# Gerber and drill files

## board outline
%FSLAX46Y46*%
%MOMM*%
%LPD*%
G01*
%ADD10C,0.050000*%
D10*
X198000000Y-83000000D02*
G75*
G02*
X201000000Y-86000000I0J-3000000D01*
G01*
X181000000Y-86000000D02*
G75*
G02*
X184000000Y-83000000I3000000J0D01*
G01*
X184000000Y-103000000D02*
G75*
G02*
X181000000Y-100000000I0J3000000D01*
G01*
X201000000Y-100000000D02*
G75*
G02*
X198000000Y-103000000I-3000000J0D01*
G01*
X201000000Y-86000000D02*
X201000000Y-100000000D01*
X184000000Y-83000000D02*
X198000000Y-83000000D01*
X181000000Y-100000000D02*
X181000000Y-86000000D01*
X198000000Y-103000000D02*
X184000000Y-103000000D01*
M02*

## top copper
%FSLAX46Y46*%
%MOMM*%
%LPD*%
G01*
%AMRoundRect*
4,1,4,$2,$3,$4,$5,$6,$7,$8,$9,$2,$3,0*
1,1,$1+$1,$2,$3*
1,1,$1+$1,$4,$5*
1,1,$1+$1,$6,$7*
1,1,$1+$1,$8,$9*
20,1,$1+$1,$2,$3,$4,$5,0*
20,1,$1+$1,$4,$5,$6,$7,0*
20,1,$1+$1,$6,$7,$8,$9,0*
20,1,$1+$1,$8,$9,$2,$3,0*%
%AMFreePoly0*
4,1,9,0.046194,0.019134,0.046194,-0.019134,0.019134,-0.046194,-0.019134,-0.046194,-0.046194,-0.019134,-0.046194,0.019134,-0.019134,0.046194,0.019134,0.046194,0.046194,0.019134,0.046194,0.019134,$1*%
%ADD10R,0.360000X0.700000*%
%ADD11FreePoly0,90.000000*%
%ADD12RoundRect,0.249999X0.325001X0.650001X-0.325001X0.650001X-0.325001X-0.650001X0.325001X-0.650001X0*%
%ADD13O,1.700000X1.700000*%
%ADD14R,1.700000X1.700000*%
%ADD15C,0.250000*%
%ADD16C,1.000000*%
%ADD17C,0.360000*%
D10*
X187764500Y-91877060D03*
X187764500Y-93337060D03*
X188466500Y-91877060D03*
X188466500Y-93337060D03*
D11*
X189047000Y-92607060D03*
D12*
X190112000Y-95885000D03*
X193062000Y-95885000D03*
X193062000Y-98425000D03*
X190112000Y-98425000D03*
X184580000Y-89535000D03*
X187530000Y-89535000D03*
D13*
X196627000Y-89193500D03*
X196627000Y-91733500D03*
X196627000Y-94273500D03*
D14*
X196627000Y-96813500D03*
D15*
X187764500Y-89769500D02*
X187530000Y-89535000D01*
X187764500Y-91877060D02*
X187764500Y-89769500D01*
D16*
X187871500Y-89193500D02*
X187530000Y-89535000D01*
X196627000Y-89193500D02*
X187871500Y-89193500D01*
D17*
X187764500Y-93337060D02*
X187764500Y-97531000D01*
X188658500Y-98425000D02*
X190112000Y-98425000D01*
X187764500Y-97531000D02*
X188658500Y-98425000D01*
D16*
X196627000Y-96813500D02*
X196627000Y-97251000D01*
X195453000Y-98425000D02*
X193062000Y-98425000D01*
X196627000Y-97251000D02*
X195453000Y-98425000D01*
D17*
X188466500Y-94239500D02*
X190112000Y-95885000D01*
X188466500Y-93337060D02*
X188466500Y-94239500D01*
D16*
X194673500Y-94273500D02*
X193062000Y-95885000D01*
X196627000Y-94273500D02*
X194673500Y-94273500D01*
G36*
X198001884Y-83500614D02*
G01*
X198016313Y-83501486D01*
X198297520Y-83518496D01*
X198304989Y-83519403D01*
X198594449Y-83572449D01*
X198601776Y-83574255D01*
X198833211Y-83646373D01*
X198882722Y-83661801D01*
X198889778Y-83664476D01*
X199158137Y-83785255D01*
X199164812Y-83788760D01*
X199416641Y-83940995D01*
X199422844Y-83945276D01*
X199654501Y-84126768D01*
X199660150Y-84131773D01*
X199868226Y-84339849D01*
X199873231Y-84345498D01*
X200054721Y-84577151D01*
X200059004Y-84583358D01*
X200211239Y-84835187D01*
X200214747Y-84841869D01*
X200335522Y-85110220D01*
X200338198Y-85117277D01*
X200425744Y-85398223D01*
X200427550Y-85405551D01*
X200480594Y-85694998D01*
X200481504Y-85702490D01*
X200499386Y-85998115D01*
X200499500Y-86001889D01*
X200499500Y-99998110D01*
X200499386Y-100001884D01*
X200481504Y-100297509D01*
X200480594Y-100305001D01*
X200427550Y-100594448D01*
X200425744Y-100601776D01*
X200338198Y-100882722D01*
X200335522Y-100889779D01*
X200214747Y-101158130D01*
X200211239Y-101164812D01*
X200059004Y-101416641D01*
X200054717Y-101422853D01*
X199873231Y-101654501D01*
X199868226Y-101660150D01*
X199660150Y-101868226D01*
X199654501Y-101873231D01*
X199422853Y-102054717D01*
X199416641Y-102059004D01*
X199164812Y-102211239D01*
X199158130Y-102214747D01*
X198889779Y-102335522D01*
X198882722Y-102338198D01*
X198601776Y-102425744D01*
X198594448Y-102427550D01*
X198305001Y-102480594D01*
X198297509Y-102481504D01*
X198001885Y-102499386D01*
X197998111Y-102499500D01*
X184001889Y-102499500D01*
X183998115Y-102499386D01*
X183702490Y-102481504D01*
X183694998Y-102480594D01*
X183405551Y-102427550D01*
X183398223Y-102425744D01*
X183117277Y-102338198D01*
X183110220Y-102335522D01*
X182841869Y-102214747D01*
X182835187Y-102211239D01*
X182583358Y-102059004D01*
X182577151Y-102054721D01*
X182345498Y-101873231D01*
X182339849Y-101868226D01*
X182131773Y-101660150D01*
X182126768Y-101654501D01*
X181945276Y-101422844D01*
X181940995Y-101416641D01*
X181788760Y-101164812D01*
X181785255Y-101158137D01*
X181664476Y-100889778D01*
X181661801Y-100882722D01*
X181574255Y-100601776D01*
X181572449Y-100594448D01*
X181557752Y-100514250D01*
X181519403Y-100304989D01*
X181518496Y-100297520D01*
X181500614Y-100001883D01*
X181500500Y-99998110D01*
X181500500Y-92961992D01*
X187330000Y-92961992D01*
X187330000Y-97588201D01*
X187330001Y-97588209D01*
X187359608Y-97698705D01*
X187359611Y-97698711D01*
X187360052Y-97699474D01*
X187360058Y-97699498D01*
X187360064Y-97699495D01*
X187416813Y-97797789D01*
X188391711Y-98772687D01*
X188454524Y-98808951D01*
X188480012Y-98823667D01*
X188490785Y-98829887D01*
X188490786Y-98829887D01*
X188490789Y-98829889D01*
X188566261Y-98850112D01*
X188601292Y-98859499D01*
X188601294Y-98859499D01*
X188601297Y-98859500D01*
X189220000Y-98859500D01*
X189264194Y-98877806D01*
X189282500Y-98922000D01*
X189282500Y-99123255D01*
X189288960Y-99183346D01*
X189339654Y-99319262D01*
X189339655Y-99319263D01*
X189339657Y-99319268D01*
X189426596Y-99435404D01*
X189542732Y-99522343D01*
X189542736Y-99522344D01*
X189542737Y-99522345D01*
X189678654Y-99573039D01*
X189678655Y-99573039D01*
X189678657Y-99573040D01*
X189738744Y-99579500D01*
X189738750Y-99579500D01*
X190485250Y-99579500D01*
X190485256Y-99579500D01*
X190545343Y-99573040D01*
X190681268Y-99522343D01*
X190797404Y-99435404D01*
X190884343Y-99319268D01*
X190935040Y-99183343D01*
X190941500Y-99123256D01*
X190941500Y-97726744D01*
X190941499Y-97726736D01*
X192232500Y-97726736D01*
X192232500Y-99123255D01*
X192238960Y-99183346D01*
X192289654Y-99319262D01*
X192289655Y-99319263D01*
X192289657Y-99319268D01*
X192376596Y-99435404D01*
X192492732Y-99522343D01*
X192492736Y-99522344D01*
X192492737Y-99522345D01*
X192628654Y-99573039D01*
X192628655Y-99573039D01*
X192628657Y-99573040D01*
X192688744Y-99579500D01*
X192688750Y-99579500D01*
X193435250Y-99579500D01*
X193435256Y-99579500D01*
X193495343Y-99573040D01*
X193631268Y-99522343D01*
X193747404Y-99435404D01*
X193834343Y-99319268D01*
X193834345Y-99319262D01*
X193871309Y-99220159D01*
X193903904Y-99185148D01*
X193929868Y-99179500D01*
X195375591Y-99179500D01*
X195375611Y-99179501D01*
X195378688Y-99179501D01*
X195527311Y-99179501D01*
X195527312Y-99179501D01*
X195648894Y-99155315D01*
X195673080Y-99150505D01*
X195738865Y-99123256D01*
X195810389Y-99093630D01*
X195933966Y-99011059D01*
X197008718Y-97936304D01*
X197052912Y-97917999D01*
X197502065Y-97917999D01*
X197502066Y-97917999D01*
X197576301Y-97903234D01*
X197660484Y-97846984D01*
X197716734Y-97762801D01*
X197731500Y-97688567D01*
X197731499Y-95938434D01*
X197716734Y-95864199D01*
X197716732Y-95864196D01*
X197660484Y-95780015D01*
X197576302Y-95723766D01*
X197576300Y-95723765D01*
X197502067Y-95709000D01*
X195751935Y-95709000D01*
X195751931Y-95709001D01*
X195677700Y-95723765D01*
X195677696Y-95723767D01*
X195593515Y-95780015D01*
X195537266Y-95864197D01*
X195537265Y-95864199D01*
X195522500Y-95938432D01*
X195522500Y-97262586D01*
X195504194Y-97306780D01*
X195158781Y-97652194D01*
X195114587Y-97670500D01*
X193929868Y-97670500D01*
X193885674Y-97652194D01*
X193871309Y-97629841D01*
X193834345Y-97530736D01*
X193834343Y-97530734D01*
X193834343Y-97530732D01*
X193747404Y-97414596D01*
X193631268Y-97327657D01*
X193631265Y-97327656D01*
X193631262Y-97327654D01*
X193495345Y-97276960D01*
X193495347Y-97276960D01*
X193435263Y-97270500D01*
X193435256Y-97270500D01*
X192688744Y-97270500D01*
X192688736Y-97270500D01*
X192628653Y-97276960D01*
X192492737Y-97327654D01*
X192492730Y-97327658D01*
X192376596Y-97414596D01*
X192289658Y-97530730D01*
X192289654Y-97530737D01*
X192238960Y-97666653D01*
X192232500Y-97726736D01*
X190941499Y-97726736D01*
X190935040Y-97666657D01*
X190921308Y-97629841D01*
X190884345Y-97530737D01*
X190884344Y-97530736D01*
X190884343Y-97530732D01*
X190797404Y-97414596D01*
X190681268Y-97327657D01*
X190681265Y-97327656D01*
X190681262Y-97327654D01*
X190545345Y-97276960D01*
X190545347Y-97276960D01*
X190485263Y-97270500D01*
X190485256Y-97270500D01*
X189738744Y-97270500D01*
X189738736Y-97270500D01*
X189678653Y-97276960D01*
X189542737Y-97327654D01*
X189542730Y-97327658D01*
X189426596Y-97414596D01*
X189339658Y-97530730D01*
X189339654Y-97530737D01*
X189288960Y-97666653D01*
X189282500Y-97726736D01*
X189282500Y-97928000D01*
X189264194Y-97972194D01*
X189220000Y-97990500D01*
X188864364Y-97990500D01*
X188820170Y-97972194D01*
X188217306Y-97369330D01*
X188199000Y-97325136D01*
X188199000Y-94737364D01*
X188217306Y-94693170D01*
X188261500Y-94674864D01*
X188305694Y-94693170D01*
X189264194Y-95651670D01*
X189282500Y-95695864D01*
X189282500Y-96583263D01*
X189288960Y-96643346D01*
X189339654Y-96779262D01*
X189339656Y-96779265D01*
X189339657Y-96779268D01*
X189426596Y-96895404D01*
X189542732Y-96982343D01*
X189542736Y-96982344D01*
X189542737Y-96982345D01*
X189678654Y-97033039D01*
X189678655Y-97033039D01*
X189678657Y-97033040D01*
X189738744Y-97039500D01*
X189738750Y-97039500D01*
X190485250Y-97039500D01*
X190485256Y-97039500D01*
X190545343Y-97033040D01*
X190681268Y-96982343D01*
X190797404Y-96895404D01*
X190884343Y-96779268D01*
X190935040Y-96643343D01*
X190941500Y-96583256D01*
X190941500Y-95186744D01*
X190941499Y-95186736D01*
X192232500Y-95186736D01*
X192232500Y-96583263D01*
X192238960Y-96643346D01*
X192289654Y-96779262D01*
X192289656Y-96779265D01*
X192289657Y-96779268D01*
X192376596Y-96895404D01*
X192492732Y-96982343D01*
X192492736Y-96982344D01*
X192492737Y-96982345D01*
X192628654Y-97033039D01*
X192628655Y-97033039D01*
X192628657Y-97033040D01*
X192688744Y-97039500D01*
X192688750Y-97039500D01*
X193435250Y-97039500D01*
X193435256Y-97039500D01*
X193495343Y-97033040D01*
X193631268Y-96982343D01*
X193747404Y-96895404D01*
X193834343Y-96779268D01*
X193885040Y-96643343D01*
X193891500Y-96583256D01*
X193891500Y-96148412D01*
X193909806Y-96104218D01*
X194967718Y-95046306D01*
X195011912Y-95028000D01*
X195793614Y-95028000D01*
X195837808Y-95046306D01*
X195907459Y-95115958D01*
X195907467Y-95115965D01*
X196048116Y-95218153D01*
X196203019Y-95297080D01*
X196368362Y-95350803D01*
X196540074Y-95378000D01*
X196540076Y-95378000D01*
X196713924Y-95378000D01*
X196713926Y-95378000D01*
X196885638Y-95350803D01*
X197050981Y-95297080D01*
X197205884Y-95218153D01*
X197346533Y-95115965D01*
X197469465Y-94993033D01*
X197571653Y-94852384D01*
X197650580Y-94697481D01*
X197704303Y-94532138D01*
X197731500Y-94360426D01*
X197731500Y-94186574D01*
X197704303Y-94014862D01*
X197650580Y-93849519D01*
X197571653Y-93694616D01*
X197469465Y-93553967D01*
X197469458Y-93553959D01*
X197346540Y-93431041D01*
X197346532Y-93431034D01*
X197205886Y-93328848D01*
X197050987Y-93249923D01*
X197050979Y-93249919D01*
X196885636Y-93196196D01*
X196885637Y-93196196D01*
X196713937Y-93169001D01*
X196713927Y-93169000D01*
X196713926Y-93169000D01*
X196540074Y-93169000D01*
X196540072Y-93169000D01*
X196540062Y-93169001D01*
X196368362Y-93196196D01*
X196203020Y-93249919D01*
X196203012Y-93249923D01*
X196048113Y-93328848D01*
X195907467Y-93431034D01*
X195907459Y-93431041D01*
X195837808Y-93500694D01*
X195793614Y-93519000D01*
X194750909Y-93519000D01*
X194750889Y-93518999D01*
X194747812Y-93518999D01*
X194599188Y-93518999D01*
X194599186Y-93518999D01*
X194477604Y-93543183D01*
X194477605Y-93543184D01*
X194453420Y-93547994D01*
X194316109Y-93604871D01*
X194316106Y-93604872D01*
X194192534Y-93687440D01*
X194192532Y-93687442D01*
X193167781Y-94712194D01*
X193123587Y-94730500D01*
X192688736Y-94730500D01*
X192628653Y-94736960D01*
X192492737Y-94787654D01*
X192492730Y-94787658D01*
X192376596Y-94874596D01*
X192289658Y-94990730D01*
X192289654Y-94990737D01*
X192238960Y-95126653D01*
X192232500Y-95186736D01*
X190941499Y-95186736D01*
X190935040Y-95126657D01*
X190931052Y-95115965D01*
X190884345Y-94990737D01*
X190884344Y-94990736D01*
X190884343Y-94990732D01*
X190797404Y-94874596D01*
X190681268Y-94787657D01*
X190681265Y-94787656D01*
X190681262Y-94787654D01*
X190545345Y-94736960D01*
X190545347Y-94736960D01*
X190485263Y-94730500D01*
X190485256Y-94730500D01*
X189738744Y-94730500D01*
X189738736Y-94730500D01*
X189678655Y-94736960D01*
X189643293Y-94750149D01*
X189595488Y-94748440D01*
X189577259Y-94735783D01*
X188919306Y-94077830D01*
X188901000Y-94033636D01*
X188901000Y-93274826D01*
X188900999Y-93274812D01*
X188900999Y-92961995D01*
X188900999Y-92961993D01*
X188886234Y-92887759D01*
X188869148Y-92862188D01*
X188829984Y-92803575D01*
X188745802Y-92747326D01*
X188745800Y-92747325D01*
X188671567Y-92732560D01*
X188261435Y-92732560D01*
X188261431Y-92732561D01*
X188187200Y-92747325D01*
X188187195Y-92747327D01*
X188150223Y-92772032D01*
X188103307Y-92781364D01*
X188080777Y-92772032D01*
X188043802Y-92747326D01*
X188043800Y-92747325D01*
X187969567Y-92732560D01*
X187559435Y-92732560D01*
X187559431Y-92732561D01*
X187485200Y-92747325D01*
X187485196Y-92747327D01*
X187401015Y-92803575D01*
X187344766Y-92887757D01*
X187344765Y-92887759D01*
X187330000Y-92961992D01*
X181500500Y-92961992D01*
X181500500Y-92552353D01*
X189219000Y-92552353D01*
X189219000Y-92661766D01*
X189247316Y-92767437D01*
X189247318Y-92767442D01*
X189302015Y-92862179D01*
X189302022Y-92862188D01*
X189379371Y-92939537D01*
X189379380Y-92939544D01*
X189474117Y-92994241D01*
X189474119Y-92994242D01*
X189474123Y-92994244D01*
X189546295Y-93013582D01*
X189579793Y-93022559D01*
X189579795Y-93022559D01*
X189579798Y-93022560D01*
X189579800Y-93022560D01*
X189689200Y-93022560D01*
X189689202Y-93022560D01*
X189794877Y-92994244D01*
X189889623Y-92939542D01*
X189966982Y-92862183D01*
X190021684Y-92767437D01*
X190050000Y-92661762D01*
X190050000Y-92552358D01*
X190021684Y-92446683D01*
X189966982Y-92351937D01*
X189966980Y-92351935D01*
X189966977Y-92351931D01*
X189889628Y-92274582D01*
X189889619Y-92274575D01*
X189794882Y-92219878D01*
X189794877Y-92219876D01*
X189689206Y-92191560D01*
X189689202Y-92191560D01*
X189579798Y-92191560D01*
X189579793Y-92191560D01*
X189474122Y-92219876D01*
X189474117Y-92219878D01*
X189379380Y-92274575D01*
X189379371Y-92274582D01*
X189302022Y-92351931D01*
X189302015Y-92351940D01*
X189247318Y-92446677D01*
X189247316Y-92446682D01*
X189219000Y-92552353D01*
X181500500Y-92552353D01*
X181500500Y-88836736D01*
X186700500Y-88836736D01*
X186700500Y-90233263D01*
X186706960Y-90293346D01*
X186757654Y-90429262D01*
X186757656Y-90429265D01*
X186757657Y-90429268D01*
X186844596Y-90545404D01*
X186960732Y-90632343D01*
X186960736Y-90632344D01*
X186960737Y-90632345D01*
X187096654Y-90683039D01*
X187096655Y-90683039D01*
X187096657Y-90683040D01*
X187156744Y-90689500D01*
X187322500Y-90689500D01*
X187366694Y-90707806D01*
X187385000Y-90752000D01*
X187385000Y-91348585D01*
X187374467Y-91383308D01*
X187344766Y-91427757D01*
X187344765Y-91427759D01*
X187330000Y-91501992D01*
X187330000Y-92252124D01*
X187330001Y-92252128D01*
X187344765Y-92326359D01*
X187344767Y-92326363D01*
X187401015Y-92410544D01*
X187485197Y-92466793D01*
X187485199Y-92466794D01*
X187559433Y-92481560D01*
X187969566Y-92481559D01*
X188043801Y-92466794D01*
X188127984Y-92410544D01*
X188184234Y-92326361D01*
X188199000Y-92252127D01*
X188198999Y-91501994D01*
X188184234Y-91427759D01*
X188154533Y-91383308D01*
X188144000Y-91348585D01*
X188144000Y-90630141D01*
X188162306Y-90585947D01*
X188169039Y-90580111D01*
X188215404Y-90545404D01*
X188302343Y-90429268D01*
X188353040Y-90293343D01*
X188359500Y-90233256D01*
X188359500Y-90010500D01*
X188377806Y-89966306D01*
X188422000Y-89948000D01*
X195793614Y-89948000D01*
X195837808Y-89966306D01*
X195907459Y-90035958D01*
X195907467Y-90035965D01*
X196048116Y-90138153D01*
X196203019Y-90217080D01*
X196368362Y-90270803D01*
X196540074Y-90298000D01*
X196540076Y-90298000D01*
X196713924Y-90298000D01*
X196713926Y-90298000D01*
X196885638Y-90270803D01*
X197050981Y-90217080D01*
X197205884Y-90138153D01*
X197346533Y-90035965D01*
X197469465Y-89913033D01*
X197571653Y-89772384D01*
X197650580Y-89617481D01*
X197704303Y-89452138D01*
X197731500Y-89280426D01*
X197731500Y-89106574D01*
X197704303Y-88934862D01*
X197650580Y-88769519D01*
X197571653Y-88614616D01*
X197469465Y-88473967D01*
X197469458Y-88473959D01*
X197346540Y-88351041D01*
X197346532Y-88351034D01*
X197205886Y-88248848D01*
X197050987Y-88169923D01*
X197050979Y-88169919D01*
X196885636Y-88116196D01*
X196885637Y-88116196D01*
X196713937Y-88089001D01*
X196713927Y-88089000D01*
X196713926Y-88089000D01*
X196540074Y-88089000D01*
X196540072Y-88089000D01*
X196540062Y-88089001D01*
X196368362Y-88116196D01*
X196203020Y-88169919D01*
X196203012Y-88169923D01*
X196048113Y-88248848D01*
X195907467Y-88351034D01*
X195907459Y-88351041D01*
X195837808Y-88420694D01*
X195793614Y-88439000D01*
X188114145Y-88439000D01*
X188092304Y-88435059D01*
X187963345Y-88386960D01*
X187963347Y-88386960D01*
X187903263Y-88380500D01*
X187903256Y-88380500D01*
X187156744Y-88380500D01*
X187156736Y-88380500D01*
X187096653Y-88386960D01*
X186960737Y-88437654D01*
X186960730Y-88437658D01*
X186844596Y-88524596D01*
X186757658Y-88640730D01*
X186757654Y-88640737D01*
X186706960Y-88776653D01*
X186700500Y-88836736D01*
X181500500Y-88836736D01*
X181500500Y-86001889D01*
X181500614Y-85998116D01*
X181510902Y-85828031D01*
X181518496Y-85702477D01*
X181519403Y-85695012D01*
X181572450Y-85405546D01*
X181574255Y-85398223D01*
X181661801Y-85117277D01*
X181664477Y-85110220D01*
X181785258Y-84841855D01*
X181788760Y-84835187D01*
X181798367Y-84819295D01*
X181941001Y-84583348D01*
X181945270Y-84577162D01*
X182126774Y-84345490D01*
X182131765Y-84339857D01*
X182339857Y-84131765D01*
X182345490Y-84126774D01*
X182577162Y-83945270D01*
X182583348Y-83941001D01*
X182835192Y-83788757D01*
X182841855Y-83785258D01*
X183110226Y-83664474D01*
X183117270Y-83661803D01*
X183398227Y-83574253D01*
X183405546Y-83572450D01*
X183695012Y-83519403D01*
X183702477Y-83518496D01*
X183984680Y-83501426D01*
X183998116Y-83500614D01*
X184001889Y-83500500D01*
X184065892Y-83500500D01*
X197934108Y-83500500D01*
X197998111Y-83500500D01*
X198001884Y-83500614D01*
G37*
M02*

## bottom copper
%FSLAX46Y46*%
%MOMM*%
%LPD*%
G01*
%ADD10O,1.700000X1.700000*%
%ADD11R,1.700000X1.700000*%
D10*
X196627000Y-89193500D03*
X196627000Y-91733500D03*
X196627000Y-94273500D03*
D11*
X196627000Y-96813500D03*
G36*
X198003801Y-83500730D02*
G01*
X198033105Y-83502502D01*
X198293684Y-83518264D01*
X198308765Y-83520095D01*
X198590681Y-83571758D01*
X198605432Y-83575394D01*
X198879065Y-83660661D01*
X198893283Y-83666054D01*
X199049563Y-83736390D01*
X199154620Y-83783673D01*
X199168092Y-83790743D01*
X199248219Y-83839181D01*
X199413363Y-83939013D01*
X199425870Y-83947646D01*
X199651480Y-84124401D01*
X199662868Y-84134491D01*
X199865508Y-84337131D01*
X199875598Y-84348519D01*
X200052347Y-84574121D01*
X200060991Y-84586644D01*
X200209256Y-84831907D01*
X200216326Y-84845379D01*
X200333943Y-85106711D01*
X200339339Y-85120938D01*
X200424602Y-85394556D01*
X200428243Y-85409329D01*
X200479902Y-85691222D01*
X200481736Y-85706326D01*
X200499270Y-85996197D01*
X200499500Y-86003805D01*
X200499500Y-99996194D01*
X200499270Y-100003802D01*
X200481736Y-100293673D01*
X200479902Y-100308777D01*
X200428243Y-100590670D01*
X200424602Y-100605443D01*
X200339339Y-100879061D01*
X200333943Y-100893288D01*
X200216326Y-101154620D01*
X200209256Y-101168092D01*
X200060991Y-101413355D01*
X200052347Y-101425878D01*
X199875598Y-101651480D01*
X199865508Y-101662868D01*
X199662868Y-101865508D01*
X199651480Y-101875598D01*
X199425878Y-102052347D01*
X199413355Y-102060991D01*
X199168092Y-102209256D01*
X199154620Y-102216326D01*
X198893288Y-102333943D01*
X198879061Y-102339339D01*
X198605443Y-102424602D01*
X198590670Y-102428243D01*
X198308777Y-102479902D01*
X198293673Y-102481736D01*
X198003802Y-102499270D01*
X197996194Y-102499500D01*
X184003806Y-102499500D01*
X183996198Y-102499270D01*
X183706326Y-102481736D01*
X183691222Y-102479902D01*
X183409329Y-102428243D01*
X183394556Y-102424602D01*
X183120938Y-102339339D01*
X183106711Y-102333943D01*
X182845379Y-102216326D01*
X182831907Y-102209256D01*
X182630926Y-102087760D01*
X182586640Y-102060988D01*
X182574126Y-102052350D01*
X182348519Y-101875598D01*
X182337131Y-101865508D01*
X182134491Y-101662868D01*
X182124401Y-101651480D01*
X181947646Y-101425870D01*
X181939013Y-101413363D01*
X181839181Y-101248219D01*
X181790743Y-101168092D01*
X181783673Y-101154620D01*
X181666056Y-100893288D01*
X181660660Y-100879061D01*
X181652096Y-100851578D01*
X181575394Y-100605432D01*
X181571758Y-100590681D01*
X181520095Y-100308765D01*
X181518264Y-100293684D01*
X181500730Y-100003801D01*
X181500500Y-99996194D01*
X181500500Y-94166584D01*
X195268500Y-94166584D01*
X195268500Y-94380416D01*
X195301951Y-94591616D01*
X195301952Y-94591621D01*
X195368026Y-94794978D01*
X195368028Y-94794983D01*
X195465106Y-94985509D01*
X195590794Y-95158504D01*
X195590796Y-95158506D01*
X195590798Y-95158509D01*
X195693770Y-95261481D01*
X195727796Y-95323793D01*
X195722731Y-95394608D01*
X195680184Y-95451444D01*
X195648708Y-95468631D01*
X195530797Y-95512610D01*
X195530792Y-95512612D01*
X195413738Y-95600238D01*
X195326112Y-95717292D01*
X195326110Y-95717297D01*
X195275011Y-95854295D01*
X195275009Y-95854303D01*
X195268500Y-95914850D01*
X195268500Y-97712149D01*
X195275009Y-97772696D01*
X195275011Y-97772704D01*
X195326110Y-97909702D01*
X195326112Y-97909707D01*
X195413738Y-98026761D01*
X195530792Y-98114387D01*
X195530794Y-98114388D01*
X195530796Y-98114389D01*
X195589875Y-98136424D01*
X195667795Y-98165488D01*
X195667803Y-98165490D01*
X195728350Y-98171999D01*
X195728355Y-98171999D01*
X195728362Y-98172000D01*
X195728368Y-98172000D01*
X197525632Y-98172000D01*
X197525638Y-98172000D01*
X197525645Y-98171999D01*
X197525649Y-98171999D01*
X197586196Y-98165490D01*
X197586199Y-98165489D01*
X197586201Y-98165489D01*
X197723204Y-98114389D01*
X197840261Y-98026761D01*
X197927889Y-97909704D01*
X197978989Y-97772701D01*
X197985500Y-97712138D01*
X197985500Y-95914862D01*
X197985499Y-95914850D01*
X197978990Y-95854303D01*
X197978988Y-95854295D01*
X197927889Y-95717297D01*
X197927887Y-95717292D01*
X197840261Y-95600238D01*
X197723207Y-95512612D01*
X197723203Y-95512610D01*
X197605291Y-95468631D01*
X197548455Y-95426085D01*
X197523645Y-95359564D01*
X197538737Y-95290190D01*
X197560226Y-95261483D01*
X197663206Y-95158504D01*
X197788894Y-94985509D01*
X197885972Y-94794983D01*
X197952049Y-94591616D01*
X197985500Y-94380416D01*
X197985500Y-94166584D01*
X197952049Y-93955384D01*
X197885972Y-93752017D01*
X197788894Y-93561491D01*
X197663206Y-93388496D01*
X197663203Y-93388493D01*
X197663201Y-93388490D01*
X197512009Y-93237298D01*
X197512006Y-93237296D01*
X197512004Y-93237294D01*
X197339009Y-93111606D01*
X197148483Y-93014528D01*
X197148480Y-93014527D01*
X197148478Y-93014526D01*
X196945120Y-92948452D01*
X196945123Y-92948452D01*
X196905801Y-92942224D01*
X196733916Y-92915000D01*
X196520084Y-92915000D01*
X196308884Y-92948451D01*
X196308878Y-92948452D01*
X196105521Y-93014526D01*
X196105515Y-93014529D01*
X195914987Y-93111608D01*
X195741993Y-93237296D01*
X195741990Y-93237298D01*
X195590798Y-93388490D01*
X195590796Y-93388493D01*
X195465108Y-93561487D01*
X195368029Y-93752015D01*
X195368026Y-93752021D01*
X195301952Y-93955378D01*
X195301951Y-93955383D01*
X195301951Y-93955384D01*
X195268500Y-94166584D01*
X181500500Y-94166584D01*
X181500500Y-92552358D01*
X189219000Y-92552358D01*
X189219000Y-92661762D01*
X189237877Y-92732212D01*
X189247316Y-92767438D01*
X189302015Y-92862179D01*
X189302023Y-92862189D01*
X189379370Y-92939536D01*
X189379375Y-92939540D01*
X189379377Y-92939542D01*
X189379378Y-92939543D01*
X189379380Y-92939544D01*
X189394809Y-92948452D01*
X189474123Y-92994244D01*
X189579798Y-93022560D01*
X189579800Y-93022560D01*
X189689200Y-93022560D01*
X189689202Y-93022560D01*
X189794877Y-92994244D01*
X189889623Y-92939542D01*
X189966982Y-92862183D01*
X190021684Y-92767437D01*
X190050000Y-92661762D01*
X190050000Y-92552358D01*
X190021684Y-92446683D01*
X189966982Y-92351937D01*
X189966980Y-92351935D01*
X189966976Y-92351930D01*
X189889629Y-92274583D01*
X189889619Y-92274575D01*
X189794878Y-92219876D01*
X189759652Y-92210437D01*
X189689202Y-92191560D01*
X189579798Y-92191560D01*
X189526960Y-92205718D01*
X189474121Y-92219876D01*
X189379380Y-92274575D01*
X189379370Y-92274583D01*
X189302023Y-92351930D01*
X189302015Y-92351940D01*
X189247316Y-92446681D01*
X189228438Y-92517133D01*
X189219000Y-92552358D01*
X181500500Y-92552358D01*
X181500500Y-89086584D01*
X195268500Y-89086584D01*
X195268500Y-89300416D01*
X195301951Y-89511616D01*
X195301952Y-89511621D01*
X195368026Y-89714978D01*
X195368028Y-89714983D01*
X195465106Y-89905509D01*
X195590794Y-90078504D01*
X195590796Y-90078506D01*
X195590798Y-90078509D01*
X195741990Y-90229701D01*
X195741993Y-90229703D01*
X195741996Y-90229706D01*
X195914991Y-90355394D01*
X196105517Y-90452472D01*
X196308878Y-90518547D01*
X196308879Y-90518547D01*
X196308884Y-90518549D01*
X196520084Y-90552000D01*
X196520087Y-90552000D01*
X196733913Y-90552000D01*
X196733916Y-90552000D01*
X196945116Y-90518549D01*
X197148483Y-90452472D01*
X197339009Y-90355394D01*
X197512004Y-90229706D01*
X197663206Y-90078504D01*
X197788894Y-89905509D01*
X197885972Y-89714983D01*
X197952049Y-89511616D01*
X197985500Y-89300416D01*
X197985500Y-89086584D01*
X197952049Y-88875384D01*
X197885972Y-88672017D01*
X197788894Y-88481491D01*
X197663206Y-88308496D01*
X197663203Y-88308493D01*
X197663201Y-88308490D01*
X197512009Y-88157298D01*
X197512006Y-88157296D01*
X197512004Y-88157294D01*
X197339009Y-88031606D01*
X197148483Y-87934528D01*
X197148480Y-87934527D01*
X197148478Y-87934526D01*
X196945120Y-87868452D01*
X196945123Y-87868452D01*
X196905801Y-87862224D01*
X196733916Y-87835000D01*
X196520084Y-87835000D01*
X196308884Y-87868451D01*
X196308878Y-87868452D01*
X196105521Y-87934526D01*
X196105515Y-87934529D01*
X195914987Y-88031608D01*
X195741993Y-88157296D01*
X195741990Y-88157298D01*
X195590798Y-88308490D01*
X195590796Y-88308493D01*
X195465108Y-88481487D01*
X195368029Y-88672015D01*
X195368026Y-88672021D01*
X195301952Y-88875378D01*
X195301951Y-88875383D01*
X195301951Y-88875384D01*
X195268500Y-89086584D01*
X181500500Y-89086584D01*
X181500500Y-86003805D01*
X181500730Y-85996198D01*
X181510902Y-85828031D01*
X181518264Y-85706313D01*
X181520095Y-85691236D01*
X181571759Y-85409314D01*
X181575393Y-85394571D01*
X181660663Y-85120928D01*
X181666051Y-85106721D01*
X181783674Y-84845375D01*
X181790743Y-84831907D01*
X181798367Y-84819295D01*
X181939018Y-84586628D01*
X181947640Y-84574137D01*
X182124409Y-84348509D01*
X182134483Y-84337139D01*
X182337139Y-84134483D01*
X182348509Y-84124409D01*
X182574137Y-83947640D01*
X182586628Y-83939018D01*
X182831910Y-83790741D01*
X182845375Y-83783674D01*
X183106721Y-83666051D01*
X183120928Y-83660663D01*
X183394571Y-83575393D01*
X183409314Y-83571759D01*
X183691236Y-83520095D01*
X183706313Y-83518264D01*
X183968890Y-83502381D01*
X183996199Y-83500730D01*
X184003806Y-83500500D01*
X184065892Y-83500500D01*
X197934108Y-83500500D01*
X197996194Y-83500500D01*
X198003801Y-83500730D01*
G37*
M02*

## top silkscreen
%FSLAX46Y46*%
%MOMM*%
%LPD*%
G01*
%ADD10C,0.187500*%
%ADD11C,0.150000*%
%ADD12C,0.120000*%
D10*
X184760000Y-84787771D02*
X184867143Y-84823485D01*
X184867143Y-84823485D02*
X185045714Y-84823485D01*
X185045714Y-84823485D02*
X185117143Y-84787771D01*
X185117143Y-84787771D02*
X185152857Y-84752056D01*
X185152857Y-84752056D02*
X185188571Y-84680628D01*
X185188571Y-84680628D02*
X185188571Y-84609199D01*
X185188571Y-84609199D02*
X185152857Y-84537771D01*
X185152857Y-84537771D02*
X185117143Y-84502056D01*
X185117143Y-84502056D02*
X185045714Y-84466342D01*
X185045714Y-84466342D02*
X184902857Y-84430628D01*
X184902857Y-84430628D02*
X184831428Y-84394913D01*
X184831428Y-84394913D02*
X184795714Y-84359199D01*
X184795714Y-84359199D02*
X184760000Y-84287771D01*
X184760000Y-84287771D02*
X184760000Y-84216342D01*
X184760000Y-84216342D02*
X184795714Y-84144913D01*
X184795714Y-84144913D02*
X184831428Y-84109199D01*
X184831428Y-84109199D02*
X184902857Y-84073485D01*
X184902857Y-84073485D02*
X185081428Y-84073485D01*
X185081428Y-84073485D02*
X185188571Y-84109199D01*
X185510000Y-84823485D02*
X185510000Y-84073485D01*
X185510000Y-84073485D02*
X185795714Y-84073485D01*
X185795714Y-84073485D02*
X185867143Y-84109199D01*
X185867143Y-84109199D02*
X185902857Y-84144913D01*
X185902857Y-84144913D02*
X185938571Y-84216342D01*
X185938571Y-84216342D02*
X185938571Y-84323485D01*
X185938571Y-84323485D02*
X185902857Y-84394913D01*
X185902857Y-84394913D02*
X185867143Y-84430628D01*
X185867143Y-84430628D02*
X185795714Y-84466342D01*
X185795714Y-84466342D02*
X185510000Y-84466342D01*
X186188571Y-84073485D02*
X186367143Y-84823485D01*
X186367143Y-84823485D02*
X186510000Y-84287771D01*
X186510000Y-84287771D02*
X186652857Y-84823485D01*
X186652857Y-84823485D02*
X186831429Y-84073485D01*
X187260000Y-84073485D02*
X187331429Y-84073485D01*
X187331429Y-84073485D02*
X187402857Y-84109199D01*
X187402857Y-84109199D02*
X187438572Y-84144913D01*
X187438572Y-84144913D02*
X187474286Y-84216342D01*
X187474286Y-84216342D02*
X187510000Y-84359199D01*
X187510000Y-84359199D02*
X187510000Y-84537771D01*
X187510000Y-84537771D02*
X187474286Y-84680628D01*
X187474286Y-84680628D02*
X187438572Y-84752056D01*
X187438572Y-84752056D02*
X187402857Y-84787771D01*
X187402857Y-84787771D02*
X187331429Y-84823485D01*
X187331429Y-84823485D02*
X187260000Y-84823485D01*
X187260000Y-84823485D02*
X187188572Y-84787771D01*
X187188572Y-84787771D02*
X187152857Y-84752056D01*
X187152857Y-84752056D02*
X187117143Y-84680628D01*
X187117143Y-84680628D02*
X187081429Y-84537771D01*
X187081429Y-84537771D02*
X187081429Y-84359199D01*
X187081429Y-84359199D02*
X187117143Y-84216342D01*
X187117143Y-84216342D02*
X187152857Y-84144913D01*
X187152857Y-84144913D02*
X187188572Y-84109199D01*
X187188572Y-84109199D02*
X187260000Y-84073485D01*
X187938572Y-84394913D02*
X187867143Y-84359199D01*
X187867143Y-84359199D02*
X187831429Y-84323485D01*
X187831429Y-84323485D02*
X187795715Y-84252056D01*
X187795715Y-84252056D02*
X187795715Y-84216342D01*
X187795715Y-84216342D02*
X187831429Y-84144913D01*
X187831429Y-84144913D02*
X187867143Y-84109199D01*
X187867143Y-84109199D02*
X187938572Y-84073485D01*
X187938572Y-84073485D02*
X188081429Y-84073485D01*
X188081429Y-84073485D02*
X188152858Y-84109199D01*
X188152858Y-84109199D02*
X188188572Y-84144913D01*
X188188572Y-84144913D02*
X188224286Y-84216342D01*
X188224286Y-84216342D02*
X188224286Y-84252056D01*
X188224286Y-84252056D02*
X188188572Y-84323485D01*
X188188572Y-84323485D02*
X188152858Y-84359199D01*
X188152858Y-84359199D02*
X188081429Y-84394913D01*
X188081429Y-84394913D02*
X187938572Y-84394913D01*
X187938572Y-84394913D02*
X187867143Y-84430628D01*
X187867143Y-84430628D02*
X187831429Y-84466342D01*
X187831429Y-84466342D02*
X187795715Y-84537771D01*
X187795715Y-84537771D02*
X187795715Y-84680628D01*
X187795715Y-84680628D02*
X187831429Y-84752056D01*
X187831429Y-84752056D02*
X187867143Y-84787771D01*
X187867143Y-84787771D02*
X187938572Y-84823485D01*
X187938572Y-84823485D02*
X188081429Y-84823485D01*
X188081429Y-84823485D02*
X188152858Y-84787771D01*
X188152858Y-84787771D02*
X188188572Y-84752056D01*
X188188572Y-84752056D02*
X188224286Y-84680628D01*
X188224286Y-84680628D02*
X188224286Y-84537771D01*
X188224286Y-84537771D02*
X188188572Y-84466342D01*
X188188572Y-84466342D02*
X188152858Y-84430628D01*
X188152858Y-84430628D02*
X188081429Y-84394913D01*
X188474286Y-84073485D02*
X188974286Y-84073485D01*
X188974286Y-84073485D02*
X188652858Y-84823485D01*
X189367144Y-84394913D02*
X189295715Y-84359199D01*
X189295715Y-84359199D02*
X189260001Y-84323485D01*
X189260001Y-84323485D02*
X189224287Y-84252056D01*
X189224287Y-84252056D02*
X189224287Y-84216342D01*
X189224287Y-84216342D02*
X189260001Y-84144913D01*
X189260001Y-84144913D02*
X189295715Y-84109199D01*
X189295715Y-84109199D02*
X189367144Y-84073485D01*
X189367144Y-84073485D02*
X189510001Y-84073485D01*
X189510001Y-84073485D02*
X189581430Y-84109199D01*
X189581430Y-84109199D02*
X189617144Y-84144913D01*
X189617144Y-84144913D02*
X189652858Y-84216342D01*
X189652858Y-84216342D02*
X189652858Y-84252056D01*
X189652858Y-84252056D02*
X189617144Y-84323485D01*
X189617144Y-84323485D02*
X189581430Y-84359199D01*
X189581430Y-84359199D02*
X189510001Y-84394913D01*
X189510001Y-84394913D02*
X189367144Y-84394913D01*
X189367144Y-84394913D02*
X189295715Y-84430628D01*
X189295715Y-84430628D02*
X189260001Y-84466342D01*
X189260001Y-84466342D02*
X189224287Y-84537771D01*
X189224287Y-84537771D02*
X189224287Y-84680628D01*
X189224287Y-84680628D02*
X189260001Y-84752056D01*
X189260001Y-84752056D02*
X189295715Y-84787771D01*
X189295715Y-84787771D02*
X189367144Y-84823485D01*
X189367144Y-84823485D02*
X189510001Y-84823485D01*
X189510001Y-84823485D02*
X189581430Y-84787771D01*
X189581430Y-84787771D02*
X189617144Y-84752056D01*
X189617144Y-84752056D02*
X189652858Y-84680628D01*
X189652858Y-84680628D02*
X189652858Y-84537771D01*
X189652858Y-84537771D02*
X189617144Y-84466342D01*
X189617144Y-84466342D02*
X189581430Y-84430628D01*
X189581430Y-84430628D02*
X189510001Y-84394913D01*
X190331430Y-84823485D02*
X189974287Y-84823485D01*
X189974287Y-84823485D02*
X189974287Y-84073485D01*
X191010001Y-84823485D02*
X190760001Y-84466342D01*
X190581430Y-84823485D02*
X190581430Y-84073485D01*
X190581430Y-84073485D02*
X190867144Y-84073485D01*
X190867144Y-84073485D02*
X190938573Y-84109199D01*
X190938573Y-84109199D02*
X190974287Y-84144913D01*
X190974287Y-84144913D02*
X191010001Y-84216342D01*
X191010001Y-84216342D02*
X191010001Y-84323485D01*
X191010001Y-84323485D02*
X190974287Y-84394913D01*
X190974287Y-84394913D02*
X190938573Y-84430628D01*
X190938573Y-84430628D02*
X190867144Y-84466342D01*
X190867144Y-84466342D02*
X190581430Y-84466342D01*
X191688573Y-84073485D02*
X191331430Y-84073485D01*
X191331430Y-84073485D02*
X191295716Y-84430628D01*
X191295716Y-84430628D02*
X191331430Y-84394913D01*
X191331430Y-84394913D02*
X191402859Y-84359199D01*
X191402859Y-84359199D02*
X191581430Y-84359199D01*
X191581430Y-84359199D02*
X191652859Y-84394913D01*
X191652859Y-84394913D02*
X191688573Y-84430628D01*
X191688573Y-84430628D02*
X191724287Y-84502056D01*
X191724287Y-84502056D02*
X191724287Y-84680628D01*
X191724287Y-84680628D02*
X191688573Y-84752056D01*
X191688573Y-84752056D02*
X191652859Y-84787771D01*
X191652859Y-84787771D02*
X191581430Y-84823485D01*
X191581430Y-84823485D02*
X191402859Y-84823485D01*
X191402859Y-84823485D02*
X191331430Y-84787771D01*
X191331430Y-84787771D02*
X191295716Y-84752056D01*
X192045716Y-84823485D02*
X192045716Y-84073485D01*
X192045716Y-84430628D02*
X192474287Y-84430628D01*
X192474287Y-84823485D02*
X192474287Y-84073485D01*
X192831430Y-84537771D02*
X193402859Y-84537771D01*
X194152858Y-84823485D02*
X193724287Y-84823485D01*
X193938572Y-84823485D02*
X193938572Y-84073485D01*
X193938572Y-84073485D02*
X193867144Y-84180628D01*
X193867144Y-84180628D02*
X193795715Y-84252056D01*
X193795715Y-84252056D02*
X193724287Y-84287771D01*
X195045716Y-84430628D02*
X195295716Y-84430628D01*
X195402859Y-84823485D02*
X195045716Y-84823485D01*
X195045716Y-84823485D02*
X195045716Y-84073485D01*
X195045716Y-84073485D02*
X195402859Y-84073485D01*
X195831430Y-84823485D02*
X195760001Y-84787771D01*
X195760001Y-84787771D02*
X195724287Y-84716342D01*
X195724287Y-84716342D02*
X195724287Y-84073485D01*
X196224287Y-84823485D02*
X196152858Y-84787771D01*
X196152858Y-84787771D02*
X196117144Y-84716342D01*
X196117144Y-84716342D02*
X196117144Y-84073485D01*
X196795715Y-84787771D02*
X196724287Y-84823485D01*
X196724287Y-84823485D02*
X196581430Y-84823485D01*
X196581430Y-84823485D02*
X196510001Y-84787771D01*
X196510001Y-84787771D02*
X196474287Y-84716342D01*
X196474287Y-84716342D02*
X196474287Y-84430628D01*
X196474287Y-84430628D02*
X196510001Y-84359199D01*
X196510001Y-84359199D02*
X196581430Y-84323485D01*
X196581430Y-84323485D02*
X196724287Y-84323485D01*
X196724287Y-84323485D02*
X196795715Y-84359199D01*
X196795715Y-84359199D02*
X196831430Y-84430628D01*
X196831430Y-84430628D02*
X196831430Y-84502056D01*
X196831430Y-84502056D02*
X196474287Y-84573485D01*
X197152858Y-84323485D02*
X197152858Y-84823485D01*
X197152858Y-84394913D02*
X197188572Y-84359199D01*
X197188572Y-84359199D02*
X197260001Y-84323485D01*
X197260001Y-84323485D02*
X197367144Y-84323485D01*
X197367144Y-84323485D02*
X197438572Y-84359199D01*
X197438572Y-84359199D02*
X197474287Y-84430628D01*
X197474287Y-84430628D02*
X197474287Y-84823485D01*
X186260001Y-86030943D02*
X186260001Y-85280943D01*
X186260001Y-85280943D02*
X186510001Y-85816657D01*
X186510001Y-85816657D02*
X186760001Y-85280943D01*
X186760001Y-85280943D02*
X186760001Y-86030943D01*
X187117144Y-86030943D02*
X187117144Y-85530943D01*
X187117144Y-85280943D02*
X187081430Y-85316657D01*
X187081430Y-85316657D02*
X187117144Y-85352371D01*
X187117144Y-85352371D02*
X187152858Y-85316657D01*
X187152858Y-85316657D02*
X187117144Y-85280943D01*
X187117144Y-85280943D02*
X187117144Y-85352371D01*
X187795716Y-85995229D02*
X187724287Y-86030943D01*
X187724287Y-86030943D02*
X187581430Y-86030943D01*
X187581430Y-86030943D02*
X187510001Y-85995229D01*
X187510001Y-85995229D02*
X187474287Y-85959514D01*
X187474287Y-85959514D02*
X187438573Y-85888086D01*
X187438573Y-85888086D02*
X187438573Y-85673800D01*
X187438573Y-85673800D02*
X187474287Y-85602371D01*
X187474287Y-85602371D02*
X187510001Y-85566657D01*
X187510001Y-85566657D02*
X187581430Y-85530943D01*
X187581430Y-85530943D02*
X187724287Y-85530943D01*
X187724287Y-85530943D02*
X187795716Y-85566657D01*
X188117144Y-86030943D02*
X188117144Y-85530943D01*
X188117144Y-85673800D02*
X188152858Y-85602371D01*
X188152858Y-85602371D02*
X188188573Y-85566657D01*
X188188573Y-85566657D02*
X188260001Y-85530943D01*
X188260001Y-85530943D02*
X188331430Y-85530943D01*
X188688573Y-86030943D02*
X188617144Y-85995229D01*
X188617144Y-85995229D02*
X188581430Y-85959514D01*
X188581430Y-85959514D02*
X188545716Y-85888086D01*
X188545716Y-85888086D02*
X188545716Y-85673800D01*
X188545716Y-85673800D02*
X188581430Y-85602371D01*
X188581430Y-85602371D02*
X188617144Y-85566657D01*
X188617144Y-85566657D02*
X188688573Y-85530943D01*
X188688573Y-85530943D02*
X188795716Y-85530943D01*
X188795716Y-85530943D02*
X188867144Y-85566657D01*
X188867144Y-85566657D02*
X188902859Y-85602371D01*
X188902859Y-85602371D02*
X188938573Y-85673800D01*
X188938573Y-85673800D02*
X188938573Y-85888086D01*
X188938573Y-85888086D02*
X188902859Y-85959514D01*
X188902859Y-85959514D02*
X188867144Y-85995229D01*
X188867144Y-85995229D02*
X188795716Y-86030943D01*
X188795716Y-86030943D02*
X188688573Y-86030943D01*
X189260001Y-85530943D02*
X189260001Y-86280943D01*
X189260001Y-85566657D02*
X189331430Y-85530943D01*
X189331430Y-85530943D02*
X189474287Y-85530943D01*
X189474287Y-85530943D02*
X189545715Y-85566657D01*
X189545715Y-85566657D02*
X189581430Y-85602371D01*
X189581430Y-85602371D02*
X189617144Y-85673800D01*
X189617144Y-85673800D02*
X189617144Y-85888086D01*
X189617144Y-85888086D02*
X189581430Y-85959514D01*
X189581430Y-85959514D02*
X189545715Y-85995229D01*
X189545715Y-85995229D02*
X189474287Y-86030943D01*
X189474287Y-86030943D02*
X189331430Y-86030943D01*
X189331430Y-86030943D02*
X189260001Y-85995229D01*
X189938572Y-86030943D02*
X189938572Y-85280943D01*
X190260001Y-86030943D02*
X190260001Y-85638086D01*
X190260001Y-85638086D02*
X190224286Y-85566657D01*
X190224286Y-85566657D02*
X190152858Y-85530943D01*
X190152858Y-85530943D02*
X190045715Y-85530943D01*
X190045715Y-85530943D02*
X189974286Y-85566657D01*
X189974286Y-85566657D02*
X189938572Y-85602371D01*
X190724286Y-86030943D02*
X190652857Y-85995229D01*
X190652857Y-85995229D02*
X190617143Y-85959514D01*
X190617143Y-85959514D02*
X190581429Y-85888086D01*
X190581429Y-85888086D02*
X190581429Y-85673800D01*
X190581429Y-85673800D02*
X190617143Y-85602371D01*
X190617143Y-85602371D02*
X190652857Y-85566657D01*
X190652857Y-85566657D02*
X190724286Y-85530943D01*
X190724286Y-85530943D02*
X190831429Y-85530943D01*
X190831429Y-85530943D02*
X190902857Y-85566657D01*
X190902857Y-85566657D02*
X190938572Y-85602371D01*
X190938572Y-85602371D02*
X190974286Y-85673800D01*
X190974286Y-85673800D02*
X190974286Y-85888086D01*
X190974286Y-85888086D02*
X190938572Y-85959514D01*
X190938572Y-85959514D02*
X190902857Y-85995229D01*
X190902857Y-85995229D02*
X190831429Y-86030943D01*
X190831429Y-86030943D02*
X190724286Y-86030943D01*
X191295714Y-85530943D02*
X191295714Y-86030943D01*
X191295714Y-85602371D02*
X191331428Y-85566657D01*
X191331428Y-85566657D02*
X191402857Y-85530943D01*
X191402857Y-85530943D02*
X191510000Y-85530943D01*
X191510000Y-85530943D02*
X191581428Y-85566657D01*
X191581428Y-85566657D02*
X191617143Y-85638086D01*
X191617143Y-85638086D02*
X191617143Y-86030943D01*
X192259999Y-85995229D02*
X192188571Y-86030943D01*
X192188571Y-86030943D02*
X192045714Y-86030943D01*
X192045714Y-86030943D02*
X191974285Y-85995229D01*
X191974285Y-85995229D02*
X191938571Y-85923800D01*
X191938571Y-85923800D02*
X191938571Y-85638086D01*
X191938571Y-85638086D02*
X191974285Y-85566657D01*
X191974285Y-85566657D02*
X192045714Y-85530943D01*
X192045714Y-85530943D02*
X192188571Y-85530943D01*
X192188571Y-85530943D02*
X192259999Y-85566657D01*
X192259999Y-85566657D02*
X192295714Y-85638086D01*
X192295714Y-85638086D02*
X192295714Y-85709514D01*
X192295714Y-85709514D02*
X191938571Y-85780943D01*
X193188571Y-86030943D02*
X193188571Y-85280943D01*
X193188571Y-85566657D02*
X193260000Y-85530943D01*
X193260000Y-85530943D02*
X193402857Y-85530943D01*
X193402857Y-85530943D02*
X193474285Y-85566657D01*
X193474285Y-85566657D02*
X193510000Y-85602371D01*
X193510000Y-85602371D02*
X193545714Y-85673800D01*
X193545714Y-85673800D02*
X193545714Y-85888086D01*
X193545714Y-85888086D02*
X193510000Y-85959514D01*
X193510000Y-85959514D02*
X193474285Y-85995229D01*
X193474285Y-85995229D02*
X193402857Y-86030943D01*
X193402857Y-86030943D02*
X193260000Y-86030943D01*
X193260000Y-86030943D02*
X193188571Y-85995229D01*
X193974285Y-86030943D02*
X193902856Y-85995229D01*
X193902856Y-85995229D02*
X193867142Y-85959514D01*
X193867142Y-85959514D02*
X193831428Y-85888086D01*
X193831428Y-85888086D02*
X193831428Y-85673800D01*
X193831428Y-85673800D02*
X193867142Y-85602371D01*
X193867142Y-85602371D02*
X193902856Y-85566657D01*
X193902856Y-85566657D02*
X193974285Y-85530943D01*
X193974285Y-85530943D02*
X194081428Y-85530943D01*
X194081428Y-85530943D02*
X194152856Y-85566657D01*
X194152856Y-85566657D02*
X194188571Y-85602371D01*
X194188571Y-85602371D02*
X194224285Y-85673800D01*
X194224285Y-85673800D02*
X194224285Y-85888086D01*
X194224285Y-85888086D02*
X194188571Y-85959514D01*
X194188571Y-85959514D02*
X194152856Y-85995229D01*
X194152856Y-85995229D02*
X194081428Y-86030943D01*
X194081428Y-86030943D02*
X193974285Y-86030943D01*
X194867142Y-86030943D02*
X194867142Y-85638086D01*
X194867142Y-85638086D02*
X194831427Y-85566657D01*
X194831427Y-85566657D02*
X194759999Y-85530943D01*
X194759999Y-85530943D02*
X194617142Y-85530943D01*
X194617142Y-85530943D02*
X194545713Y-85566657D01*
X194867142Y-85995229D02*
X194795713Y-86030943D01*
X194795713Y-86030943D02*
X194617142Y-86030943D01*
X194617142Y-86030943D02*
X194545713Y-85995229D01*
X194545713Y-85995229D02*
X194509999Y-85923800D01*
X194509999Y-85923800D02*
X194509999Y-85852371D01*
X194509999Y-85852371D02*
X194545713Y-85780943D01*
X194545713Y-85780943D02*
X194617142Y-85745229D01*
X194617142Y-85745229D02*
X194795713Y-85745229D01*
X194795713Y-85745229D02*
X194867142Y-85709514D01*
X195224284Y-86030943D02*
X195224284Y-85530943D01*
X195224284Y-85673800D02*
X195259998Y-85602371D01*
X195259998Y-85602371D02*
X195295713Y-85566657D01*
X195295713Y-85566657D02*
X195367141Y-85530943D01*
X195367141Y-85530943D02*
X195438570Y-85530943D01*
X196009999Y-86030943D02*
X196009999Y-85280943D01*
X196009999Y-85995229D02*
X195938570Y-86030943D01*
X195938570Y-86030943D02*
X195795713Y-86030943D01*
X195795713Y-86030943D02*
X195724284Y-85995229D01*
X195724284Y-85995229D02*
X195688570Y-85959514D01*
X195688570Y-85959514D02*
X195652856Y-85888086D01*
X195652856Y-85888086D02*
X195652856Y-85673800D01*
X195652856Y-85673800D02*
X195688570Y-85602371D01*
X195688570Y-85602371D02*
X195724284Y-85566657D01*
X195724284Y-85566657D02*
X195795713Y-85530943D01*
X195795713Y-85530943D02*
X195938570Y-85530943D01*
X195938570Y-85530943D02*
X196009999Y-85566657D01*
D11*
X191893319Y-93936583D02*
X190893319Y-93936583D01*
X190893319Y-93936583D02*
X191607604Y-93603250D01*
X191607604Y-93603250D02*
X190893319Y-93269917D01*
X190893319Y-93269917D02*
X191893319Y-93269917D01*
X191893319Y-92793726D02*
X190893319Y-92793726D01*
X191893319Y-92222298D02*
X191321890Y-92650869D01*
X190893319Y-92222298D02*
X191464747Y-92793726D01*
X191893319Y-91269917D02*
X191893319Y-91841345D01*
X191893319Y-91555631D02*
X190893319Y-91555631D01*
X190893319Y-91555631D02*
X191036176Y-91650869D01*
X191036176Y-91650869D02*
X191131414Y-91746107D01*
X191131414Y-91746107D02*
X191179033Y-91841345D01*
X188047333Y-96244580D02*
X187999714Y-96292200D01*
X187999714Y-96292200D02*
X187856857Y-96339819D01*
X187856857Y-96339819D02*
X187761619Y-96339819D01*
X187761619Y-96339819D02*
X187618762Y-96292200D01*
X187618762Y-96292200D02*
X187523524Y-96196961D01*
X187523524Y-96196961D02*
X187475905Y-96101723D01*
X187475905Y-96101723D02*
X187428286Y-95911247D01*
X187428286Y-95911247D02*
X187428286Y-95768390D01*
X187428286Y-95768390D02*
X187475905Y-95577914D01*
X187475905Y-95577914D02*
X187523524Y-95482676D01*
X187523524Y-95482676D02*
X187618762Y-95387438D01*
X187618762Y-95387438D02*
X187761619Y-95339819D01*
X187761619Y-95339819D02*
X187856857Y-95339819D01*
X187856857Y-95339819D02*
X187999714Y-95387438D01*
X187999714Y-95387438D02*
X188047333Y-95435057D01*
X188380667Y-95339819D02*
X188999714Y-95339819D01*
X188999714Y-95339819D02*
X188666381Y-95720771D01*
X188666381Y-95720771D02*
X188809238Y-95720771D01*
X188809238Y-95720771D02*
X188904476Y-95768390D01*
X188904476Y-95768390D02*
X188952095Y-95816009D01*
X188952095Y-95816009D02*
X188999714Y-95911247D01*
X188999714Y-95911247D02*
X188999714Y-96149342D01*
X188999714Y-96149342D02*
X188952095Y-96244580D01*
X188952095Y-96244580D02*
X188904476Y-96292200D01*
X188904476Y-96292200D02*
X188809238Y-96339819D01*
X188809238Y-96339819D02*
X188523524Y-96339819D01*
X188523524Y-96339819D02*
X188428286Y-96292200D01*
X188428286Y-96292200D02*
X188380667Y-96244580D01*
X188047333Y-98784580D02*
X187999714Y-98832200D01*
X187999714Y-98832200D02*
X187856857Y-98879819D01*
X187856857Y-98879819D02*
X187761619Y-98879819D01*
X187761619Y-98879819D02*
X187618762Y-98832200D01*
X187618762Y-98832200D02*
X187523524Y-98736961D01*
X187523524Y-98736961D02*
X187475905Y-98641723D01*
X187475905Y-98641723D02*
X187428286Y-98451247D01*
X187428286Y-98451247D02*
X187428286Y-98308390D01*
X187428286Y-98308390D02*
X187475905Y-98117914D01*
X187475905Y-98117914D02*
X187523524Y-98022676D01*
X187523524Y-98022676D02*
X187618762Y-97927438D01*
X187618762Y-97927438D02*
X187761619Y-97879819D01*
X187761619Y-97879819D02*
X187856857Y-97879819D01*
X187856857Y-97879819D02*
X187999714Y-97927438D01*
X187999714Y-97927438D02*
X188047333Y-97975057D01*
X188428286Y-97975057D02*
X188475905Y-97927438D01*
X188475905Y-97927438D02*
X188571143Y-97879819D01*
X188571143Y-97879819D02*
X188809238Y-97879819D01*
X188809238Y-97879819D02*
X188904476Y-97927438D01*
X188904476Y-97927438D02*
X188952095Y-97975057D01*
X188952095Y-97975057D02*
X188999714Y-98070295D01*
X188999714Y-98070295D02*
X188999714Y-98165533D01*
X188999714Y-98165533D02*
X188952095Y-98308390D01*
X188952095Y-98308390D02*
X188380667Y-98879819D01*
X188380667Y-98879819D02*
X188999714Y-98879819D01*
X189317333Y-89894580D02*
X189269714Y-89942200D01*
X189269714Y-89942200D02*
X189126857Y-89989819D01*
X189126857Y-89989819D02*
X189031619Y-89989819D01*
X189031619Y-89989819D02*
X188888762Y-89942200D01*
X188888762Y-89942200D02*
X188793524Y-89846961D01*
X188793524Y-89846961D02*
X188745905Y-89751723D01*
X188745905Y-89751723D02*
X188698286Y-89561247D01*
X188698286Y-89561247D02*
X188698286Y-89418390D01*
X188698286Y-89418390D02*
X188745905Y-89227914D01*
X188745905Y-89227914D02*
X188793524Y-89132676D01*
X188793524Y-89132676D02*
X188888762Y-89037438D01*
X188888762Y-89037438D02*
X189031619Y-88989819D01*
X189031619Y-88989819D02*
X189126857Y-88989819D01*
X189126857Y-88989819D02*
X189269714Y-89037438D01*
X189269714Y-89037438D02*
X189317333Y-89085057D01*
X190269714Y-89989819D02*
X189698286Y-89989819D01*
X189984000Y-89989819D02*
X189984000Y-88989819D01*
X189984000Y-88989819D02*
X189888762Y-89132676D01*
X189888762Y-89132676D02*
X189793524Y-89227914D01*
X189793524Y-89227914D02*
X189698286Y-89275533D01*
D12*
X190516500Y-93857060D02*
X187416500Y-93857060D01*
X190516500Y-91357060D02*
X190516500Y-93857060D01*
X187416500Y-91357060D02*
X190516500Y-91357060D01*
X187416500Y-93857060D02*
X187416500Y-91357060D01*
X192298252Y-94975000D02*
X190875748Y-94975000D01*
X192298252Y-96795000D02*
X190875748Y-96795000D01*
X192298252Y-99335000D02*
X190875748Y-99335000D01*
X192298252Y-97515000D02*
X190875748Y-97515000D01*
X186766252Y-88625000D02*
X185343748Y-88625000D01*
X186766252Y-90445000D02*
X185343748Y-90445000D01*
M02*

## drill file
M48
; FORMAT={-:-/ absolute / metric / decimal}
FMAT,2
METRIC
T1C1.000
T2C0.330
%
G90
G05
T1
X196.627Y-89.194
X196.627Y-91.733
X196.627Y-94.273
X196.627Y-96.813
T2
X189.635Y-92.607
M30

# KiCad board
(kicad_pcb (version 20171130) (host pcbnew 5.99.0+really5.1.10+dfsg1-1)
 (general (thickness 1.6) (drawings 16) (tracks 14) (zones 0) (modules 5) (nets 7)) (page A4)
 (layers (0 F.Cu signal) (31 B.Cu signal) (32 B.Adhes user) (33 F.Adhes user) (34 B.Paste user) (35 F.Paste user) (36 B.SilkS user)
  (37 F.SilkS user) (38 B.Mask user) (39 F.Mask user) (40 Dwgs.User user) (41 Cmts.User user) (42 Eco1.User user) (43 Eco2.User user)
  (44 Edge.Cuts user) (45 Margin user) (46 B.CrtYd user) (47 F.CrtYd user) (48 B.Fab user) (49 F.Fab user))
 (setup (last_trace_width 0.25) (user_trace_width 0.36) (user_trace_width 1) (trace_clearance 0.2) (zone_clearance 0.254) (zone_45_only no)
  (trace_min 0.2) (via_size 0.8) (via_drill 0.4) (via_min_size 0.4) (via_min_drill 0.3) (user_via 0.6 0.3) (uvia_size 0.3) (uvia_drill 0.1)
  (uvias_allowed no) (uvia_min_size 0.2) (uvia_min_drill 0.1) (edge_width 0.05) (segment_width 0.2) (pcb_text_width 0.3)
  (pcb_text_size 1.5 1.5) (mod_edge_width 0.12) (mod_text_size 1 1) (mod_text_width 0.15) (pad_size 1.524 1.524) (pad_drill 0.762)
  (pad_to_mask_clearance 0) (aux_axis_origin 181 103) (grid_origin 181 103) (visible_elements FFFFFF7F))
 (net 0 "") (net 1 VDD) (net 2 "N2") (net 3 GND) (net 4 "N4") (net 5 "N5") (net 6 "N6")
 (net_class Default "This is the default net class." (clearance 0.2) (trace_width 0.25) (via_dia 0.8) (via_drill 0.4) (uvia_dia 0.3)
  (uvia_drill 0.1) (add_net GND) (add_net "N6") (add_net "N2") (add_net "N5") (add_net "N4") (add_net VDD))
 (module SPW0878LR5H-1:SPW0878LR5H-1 (layer F.Cu) (at 188.9665 92.60706 90)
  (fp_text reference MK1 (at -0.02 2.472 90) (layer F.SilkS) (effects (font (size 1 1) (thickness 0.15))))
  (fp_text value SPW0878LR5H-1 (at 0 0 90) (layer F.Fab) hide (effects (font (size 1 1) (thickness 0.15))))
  (fp_line (start -1.25 1.55) (end -1.25 -1.55) (layer F.SilkS) (width 0.12))
  (fp_line (start 1.25 1.55) (end -1.25 1.55) (layer F.SilkS) (width 0.12))
  (fp_line (start 1.25 -1.55) (end 1.25 1.55) (layer F.SilkS) (width 0.12))
  (fp_line (start -1.25 -1.55) (end 1.25 -1.55) (layer F.SilkS) (width 0.12))
  (pad 5 smd rect (at 0.73 -1.202 90) (size 0.7 0.36) (layers F.Cu F.Paste F.Mask) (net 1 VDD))
  (pad 1 smd rect (at -0.73 -1.202 90) (size 0.7 0.36) (layers F.Cu F.Paste F.Mask) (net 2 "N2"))
  (pad 4 smd rect (at 0.73 -0.5 90) (size 0.7 0.36) (layers F.Cu F.Paste F.Mask) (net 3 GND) (zone_connect 2))
  (pad 2 smd rect (at -0.73 -0.5 90) (size 0.7 0.36) (layers F.Cu F.Paste F.Mask) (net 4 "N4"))
  (pad 3 smd custom (at 0 0.0805 90) (size 0.1 0.1) (layers F.Cu F.Paste F.Mask) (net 3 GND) (zone_connect 2)
   (options (clearance outline) (anchor circle)) (primitives))
  (pad "" np_thru_hole circle (at 0 0.668 90) (size 0.33 0.33) (drill 0.33) (layers *.Cu *.Mask)))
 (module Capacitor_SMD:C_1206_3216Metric (layer F.Cu) (at 191.587 95.885 180)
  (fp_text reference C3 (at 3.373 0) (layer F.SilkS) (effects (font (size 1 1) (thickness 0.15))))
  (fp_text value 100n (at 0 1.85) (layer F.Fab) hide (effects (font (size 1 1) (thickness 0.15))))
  (fp_line (start -0.711252 0.91) (end 0.711252 0.91) (layer F.SilkS) (width 0.12))
  (fp_line (start -0.711252 -0.91) (end 0.711252 -0.91) (layer F.SilkS) (width 0.12))
  (pad 2 smd roundrect (at 1.475 0 180) (size 1.15 1.8) (layers F.Cu F.Paste F.Mask) (roundrect_rratio 0.2173904347826087) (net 4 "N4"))
  (pad 1 smd roundrect (at -1.475 0 180) (size 1.15 1.8) (layers F.Cu F.Paste F.Mask) (roundrect_rratio 0.2173904347826087) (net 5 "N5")))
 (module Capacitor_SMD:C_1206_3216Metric (layer F.Cu) (at 191.587 98.425 180)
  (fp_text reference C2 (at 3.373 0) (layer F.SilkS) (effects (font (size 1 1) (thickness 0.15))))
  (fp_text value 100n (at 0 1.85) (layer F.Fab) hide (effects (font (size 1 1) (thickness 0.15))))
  (fp_line (start -0.711252 -0.91) (end 0.711252 -0.91) (layer F.SilkS) (width 0.12))
  (fp_line (start -0.711252 0.91) (end 0.711252 0.91) (layer F.SilkS) (width 0.12))
  (pad 1 smd roundrect (at -1.475 0 180) (size 1.15 1.8) (layers F.Cu F.Paste F.Mask) (roundrect_rratio 0.2173904347826087) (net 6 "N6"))
  (pad 2 smd roundrect (at 1.475 0 180) (size 1.15 1.8) (layers F.Cu F.Paste F.Mask) (roundrect_rratio 0.2173904347826087) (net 2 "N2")))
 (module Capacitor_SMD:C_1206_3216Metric (layer F.Cu) (at 186.055 89.535 180)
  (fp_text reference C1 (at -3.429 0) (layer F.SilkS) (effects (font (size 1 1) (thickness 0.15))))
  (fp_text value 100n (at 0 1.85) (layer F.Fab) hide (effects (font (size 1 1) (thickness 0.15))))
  (fp_line (start -0.711252 0.91) (end 0.711252 0.91) (layer F.SilkS) (width 0.12))
  (fp_line (start -0.711252 -0.91) (end 0.711252 -0.91) (layer F.SilkS) (width 0.12))
  (pad 2 smd roundrect (at 1.475 0 180) (size 1.15 1.8) (layers F.Cu F.Paste F.Mask) (roundrect_rratio 0.2173904347826087) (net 3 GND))
  (pad 1 smd roundrect (at -1.475 0 180) (size 1.15 1.8) (layers F.Cu F.Paste F.Mask) (roundrect_rratio 0.2173904347826087) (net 1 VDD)))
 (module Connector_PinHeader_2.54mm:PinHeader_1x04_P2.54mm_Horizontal (layer B.Cu) (at 196.627 96.8135)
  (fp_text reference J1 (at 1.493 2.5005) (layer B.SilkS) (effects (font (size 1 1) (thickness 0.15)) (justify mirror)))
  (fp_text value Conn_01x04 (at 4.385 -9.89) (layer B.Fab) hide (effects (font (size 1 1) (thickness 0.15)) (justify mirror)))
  (pad 4 thru_hole oval (at 0 -7.62) (size 1.7 1.7) (drill 1) (layers *.Cu *.Mask) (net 1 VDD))
  (pad 3 thru_hole oval (at 0 -5.08) (size 1.7 1.7) (drill 1) (layers *.Cu *.Mask) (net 3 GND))
  (pad 2 thru_hole oval (at 0 -2.54) (size 1.7 1.7) (drill 1) (layers *.Cu *.Mask) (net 5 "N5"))
  (pad 1 thru_hole rect (at 0 0) (size 1.7 1.7) (drill 1) (layers *.Cu *.Mask) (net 6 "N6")))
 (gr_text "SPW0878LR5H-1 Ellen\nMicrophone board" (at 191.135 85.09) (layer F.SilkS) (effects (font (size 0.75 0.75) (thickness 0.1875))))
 (gr_arc (start 198 86) (end 201 86) (angle -90) (layer Edge.Cuts) (width 0.05))
 (gr_arc (start 184 86) (end 184 83) (angle -90) (layer Edge.Cuts) (width 0.05))
 (gr_arc (start 184 100) (end 181 100) (angle -90) (layer Edge.Cuts) (width 0.05))
 (gr_arc (start 198 100) (end 198 103) (angle -90) (layer Edge.Cuts) (width 0.05))
 (gr_line (start 201 86) (end 201 100) (layer Edge.Cuts) (width 0.05))
 (gr_line (start 184 83) (end 198 83) (layer Edge.Cuts) (width 0.05))
 (gr_line (start 181 100) (end 181 86) (layer Edge.Cuts) (width 0.05))
 (gr_line (start 198 103) (end 184 103) (layer Edge.Cuts) (width 0.05))
 (segment (start 187.7645 89.7695) (end 187.53 89.535) (width 0.25) (layer F.Cu) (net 1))
 (segment (start 187.7645 91.87706) (end 187.7645 89.7695) (width 0.25) (layer F.Cu) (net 1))
 (segment (start 187.8715 89.1935) (end 187.53 89.535) (width 1) (layer F.Cu) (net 1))
 (segment (start 196.627 89.1935) (end 187.8715 89.1935) (width 1) (layer F.Cu) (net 1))
 (segment (start 187.7645 93.33706) (end 187.7645 97.531) (width 0.36) (layer F.Cu) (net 2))
 (segment (start 188.6585 98.425) (end 190.112 98.425) (width 0.36) (layer F.Cu) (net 2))
 (segment (start 187.7645 97.531) (end 188.6585 98.425) (width 0.36) (layer F.Cu) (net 2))
 (segment (start 196.627 96.8135) (end 196.627 97.251) (width 1) (layer F.Cu) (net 6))
 (segment (start 195.453 98.425) (end 193.062 98.425) (width 1) (layer F.Cu) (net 6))
 (segment (start 196.627 97.251) (end 195.453 98.425) (width 1) (layer F.Cu) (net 6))
 (segment (start 188.4665 94.2395) (end 190.112 95.885) (width 0.36) (layer F.Cu) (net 4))
 (segment (start 188.4665 93.33706) (end 188.4665 94.2395) (width 0.36) (layer F.Cu) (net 4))
 (segment (start 194.6735 94.2735) (end 193.062 95.885) (width 1) (layer F.Cu) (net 5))
 (segment (start 196.627 94.2735) (end 194.6735 94.2735) (width 1) (layer F.Cu) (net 5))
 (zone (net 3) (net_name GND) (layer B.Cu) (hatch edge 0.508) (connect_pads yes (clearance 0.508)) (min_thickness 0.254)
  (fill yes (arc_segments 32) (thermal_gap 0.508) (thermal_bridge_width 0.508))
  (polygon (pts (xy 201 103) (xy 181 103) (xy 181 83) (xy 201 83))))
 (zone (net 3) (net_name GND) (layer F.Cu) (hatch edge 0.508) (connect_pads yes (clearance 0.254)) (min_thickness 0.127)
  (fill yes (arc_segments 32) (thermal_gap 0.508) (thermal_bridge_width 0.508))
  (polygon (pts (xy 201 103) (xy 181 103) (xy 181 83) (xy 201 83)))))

